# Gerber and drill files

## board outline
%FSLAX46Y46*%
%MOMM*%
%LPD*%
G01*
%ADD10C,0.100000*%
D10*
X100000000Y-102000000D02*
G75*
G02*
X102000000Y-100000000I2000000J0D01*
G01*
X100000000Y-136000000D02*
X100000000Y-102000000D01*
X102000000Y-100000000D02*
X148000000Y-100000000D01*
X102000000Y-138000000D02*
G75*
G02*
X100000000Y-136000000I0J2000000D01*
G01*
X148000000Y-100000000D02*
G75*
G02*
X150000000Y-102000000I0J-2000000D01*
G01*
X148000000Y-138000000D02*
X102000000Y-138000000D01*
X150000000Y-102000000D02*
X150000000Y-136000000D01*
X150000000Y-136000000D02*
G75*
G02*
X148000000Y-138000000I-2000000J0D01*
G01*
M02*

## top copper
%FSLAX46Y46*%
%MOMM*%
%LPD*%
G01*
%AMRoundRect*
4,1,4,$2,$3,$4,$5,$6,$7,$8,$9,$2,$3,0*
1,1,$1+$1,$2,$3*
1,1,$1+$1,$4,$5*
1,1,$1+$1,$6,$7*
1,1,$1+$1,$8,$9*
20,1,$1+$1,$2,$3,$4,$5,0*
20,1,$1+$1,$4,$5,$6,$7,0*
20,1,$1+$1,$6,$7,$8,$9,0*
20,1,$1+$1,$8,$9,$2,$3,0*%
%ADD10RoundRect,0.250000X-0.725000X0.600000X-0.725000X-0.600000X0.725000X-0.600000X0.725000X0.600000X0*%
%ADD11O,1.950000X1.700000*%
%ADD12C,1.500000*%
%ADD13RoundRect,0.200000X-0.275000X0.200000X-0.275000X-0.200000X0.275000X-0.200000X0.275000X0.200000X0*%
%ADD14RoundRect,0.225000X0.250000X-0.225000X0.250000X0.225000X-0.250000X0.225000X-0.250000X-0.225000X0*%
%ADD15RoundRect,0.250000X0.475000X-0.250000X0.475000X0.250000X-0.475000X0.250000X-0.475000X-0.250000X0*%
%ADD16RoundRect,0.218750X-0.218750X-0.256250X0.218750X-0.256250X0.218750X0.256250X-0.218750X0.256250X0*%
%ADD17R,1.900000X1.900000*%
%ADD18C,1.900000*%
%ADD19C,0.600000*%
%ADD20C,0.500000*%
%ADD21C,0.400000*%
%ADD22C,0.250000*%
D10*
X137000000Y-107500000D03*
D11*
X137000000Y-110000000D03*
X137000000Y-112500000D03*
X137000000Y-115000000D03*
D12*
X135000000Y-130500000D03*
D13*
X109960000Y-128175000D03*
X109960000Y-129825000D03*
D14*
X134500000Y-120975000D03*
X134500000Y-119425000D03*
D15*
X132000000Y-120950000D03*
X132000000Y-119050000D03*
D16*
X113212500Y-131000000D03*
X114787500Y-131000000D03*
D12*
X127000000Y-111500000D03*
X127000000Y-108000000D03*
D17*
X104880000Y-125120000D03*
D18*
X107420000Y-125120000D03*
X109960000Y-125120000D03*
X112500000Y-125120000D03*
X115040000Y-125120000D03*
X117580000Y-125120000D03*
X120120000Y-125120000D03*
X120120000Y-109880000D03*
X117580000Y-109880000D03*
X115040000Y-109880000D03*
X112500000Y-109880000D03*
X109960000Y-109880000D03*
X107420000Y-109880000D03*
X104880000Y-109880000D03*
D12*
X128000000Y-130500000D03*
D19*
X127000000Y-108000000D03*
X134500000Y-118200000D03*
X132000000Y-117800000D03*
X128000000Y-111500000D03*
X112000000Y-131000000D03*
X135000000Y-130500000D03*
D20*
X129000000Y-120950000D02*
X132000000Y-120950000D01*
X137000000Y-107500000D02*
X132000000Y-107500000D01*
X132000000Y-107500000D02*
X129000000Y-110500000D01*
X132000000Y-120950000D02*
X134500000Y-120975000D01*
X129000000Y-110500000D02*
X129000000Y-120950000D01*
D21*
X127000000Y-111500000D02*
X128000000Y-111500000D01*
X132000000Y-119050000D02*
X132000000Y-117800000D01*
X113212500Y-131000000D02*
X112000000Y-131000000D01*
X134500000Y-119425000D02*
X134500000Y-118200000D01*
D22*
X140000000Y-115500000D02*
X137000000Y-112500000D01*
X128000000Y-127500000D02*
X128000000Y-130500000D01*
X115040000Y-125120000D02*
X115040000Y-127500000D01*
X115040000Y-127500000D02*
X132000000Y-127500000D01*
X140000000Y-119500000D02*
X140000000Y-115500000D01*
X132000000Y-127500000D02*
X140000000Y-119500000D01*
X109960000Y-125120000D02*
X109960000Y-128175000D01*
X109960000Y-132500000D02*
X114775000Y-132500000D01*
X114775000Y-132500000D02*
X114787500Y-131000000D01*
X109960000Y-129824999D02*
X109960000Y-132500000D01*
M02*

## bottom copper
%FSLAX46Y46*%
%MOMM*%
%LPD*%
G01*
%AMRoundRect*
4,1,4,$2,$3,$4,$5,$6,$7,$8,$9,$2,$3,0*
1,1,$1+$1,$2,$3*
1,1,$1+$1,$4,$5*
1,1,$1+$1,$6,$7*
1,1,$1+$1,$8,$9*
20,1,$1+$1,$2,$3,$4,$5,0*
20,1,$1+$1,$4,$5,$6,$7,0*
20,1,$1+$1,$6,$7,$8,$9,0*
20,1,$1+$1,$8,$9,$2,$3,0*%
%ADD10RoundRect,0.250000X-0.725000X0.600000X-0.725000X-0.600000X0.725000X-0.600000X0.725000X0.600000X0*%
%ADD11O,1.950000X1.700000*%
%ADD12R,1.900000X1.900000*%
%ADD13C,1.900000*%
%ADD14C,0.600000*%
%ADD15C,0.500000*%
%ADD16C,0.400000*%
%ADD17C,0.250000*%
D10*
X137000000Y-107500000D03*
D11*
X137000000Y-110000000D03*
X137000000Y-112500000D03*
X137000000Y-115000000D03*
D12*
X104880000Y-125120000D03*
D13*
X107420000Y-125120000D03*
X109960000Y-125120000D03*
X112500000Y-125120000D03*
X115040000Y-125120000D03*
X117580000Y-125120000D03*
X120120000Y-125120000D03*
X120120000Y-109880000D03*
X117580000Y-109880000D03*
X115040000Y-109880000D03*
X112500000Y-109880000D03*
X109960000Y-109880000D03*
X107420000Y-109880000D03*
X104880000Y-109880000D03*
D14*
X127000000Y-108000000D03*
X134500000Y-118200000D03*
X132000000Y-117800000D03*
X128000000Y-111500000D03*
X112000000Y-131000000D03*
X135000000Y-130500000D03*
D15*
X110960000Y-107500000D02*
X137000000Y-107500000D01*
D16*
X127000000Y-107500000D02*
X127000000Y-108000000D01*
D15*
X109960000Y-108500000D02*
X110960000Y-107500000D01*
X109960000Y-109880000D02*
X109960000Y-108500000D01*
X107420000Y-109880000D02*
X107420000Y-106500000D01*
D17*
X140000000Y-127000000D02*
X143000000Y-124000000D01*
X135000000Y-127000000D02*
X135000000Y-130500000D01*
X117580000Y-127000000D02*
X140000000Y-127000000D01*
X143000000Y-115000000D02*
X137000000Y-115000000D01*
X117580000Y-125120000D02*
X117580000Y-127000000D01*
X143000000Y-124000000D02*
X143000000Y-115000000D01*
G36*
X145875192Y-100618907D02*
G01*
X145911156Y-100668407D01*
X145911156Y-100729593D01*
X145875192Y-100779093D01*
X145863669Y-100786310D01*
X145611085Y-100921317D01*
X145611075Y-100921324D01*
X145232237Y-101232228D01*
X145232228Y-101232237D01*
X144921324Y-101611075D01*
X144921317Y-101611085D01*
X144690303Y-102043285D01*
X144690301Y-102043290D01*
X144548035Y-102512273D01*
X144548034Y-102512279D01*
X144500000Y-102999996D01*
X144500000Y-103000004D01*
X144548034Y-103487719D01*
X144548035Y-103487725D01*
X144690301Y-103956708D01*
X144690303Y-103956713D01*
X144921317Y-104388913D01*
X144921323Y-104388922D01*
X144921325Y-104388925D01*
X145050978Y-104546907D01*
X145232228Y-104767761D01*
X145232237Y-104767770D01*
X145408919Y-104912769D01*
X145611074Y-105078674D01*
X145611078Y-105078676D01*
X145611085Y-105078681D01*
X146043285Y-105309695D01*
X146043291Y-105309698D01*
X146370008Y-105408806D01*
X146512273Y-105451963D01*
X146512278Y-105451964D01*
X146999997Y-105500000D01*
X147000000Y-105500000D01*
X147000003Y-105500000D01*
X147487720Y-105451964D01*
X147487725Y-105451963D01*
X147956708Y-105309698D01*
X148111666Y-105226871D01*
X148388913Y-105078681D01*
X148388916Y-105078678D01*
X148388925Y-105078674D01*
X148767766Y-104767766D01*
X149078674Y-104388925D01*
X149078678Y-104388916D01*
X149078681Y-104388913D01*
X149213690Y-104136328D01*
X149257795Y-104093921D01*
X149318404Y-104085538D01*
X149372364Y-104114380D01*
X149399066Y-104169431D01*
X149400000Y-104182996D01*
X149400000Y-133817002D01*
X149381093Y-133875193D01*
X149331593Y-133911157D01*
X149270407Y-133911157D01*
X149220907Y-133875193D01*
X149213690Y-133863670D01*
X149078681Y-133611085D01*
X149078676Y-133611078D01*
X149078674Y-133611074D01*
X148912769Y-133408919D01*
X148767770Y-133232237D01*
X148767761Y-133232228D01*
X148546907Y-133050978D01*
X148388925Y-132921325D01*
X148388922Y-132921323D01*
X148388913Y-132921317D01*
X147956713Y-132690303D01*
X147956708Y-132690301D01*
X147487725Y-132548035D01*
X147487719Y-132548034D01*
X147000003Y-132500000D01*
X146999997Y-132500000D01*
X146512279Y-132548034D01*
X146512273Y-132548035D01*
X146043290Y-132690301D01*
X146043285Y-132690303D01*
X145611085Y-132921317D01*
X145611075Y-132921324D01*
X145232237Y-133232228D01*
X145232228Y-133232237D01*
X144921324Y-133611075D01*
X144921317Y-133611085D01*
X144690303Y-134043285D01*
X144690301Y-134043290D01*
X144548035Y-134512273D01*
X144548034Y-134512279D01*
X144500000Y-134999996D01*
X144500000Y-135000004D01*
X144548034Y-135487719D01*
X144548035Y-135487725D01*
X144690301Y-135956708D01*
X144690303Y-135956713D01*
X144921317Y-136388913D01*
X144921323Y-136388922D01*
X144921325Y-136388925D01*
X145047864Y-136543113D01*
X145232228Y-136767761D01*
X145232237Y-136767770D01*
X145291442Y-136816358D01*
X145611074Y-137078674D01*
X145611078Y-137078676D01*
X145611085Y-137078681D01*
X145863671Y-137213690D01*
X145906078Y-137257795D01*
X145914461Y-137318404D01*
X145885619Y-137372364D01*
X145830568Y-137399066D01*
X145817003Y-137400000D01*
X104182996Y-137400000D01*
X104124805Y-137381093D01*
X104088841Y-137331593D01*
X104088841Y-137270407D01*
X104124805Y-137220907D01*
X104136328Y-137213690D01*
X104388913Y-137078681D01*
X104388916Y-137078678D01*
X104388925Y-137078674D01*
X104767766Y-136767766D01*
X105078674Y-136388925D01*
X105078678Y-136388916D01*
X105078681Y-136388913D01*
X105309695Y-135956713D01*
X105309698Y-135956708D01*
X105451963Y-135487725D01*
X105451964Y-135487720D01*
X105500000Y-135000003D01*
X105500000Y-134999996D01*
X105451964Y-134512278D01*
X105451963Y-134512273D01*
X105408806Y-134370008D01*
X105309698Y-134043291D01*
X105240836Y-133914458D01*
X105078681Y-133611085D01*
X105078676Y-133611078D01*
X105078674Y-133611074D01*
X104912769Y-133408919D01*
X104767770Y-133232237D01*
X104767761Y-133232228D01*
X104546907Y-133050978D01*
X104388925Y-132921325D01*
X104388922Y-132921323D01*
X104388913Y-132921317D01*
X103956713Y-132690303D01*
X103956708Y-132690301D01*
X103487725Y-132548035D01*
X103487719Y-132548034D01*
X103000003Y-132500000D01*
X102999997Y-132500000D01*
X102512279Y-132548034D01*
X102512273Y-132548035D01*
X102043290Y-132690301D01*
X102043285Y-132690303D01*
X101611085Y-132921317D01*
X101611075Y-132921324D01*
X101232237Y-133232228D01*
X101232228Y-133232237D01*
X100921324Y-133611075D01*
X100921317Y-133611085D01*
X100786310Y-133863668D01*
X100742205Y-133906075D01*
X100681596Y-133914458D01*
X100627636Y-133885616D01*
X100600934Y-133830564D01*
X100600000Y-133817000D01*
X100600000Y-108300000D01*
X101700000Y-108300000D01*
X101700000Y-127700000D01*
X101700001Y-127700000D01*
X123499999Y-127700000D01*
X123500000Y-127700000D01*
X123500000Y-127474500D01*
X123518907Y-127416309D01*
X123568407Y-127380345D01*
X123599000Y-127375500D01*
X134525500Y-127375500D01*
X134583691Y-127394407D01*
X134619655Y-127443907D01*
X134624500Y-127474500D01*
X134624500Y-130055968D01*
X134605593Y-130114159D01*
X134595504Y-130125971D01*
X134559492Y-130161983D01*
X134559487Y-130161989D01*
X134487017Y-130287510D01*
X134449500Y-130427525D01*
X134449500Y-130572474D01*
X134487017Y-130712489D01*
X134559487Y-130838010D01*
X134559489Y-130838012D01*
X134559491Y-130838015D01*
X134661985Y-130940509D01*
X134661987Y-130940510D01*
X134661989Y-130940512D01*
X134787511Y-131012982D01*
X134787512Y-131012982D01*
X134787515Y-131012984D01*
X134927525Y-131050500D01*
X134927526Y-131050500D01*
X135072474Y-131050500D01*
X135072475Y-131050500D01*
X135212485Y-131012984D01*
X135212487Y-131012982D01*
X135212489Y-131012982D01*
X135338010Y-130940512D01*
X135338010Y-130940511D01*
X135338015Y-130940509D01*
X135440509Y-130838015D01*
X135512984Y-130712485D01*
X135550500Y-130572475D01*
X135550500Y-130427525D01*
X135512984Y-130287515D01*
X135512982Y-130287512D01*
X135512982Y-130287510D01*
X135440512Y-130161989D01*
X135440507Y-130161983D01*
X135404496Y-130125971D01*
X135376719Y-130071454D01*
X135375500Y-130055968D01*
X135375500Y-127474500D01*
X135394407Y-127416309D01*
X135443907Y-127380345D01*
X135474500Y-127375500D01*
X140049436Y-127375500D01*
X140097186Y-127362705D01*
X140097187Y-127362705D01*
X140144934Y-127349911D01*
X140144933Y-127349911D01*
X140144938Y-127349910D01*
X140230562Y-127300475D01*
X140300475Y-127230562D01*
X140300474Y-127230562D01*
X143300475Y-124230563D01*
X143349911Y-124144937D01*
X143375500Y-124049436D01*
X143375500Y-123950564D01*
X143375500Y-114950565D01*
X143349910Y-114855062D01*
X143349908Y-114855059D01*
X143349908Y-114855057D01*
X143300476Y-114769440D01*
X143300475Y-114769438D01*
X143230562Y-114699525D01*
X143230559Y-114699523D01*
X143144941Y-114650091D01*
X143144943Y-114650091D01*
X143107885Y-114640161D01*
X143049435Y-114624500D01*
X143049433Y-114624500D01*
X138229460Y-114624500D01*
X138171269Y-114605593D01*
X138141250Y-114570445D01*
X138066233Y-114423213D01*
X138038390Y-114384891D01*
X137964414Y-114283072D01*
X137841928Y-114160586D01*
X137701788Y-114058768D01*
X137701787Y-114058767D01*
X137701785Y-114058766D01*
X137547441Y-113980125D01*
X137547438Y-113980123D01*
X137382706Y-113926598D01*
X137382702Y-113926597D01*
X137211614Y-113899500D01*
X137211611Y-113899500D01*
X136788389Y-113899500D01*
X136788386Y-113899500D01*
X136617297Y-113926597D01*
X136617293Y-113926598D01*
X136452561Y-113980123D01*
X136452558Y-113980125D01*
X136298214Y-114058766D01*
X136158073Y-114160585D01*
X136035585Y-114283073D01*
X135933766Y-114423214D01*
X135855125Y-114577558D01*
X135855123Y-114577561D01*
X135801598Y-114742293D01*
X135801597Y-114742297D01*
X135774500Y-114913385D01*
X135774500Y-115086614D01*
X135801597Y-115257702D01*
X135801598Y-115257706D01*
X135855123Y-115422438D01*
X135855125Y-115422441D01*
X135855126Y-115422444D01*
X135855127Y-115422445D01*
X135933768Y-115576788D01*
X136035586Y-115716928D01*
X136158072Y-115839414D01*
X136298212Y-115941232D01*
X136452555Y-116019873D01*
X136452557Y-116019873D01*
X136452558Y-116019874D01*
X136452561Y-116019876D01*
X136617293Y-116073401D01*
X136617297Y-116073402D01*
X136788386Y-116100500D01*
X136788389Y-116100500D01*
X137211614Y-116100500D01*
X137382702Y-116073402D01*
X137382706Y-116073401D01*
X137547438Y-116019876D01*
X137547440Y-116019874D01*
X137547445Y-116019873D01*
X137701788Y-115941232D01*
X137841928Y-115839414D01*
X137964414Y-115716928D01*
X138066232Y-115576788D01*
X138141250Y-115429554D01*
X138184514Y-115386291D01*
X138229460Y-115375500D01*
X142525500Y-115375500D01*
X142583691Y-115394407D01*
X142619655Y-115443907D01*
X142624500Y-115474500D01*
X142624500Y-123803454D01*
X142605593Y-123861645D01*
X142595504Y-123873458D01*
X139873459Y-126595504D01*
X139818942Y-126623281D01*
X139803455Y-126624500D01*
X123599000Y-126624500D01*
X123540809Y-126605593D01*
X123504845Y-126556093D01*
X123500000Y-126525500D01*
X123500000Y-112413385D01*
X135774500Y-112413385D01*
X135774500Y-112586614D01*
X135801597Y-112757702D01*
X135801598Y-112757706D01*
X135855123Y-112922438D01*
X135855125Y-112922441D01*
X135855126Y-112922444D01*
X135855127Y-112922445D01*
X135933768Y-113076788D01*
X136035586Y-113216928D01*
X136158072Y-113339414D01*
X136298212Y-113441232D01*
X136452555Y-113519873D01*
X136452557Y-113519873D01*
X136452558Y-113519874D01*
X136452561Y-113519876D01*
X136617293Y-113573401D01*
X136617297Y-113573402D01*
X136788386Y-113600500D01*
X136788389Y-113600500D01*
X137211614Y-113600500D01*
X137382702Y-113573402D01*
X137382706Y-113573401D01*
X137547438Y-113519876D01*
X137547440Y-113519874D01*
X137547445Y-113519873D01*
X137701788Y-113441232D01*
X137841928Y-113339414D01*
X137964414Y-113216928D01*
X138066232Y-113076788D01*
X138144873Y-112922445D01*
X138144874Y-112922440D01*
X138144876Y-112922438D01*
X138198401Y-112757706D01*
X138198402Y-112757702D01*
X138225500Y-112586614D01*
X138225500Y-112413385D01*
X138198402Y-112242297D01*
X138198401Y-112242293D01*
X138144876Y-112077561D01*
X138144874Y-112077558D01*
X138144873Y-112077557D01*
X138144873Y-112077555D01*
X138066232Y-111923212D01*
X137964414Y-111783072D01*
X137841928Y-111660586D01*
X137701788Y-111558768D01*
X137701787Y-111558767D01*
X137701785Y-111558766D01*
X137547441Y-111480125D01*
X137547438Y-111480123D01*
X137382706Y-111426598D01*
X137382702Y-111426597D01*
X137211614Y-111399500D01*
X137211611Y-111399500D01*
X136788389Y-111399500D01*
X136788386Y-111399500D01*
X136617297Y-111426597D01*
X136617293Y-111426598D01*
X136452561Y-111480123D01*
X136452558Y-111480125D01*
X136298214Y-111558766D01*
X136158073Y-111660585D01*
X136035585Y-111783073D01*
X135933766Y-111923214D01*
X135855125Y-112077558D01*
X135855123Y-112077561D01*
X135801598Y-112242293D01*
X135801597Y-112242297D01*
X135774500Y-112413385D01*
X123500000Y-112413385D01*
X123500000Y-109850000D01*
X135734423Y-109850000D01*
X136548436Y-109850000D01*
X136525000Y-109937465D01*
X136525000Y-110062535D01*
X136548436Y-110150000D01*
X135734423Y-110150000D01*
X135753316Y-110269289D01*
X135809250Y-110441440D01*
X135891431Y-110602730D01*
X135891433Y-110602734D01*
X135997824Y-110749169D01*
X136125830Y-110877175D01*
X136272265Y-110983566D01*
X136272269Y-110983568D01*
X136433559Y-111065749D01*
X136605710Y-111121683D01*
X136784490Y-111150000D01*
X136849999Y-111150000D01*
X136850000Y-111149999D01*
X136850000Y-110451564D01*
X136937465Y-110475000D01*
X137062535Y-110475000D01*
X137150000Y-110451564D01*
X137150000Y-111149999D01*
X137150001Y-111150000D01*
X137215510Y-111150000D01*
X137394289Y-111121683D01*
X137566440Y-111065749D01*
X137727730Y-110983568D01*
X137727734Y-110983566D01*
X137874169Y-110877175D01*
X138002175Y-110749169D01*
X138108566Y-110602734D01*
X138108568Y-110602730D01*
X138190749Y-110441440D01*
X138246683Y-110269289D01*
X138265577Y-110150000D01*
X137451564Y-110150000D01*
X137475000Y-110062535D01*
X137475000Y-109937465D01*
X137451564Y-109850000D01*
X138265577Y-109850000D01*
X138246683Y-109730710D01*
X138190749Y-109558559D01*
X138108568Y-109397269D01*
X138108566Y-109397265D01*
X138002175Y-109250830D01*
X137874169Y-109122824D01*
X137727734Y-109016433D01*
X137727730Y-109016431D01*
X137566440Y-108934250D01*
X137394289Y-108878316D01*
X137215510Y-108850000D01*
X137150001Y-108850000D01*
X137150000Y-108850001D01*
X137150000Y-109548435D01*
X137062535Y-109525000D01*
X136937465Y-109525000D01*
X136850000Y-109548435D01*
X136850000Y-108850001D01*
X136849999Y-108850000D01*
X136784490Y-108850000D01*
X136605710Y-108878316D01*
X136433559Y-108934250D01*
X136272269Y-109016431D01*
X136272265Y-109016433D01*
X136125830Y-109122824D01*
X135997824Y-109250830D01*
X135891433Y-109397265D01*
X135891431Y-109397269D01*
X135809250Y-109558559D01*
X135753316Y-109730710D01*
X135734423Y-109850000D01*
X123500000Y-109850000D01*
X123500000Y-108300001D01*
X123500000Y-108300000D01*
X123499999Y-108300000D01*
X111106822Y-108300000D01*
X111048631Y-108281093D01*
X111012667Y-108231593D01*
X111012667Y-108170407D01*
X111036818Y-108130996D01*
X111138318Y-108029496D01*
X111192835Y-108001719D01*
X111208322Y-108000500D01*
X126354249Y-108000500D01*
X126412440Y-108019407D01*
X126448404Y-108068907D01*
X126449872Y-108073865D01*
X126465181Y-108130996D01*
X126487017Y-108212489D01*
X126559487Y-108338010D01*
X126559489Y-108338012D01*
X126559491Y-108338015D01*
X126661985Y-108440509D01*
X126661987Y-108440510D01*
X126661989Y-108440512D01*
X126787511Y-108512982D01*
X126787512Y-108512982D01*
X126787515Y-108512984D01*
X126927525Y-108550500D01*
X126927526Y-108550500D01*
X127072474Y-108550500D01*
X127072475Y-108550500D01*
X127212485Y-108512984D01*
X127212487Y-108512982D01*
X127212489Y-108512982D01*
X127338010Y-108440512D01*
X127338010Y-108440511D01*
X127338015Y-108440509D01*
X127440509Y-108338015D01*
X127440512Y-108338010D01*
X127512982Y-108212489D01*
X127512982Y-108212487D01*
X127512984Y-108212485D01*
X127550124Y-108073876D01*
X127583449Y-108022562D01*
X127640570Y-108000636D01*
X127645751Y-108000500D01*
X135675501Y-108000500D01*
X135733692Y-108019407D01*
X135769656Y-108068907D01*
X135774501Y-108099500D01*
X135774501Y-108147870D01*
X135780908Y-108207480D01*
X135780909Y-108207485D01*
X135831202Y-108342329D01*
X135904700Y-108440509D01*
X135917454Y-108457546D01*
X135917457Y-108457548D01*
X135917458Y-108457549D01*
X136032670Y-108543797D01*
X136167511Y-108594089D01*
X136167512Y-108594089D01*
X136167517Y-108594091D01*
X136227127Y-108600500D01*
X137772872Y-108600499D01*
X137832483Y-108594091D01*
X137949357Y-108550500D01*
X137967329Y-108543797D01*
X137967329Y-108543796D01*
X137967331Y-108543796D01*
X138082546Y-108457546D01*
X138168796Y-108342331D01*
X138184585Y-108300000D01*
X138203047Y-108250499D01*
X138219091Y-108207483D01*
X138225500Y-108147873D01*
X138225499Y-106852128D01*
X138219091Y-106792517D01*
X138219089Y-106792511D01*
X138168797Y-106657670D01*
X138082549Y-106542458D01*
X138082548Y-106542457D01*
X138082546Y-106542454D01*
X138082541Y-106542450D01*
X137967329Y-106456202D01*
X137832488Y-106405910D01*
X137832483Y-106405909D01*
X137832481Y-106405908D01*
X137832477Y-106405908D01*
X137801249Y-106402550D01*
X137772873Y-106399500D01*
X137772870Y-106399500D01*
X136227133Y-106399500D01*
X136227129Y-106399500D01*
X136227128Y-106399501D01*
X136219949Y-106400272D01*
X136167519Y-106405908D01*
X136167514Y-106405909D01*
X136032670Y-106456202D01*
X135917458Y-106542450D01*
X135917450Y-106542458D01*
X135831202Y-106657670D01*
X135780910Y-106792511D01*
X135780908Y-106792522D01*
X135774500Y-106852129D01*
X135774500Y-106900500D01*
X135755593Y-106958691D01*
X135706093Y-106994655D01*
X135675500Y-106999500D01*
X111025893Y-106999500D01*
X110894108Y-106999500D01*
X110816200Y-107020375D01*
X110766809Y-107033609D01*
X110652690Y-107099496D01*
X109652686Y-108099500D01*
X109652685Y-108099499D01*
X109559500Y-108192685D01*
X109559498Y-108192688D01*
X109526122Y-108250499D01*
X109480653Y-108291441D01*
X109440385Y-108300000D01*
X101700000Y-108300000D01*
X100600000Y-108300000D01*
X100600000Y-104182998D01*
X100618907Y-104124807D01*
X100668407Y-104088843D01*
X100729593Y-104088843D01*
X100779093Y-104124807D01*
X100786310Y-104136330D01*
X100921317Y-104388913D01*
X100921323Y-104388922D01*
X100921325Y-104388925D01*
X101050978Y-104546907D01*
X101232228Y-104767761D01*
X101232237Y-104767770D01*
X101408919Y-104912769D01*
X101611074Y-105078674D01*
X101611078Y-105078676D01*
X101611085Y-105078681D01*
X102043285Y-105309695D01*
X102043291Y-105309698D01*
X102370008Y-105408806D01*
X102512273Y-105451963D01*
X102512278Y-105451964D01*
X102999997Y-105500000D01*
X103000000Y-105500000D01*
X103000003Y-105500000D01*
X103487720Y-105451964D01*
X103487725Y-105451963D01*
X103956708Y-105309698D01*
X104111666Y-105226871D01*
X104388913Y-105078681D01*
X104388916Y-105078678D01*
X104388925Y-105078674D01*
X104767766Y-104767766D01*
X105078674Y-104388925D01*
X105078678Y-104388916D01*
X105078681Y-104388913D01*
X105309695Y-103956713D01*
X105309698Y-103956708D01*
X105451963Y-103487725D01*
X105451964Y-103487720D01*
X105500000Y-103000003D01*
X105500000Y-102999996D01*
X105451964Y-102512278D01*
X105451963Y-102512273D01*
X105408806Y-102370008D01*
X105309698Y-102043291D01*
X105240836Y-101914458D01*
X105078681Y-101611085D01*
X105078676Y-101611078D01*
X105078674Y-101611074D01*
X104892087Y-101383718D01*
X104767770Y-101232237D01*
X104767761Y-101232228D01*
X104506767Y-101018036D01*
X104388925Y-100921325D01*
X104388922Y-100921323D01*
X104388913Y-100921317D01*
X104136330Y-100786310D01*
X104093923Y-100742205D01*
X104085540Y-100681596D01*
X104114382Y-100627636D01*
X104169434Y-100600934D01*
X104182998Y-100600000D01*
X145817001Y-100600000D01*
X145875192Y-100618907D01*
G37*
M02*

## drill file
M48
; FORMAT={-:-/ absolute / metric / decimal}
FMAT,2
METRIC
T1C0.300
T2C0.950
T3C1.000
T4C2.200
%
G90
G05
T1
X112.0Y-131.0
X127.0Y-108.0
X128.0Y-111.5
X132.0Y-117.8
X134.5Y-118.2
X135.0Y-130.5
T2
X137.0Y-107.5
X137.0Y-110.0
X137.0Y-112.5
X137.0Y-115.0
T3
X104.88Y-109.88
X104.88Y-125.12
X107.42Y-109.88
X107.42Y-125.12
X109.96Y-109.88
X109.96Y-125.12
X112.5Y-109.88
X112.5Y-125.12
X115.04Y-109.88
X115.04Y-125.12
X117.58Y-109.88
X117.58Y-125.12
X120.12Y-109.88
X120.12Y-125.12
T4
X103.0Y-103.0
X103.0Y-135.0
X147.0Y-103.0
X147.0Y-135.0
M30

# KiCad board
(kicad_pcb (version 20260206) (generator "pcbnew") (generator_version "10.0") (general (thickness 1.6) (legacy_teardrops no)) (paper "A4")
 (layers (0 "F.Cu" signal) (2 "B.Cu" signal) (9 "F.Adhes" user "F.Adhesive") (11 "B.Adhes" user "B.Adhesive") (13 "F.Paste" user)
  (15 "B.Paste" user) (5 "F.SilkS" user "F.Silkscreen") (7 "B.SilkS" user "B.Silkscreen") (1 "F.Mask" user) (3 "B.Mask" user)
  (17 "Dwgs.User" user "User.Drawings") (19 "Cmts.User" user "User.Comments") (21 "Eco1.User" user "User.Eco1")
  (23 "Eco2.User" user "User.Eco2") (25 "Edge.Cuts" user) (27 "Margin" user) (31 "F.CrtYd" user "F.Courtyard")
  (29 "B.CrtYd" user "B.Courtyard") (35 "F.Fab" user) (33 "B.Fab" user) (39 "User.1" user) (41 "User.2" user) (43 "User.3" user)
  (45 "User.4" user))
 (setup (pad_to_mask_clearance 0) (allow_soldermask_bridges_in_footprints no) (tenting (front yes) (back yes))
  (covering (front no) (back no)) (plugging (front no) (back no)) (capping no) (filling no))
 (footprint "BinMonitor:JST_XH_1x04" (layer "F.Cu") (at 137 107.5 -90)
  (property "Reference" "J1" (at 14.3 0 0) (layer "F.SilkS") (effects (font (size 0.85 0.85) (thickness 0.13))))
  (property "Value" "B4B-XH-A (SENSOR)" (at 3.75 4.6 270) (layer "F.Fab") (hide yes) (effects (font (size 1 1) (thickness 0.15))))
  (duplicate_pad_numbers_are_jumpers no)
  (pad "1" thru_hole roundrect (at 0 0 270) (size 1.7 1.95) (drill 0.95) (layers "*.Cu" "*.Mask") (remove_unused_layers no)
   (roundrect_rratio 0.147059) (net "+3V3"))
  (pad "2" thru_hole oval (at 2.5 0 270) (size 1.7 1.95) (drill 0.95) (layers "*.Cu" "*.Mask") (remove_unused_layers no) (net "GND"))
  (pad "3" thru_hole oval (at 5 0 270) (size 1.7 1.95) (drill 0.95) (layers "*.Cu" "*.Mask") (remove_unused_layers no) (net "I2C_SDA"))
  (pad "4" thru_hole oval (at 7.5 0 270) (size 1.7 1.95) (drill 0.95) (layers "*.Cu" "*.Mask") (remove_unused_layers no) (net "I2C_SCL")))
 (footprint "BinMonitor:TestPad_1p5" (layer "F.Cu") (at 135 130.5)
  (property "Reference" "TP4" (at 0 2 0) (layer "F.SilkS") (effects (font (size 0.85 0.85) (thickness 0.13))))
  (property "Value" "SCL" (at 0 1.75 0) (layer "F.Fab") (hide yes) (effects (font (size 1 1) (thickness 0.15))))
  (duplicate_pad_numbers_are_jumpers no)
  (pad "1" smd circle (at 0 0) (size 1.5 1.5) (layers "F.Cu" "F.Mask") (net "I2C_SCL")))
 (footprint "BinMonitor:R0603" (layer "F.Cu") (at 109.96 129 -90)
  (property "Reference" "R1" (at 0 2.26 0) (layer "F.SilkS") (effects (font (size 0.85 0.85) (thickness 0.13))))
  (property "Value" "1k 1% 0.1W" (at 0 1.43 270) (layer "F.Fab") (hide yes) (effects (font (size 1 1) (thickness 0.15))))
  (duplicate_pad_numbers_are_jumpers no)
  (pad "1" smd roundrect (at -0.825 0 270) (size 0.8 0.95) (layers "F.Cu" "F.Mask" "F.Paste") (roundrect_rratio 0.25) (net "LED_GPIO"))
  (pad "2" smd roundrect (at 0.825 0 270) (size 0.8 0.95) (layers "F.Cu" "F.Mask" "F.Paste") (roundrect_rratio 0.25) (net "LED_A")))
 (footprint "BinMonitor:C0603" (layer "F.Cu") (at 134.5 120.2 90)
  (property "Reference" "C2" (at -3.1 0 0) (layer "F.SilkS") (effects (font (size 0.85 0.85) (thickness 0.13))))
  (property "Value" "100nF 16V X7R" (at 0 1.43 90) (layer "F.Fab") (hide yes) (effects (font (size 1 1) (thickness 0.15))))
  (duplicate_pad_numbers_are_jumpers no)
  (pad "1" smd roundrect (at -0.775 0 90) (size 0.9 0.95) (layers "F.Cu" "F.Mask" "F.Paste") (roundrect_rratio 0.25) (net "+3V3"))
  (pad "2" smd roundrect (at 0.775 0 90) (size 0.9 0.95) (layers "F.Cu" "F.Mask" "F.Paste") (roundrect_rratio 0.25) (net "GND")))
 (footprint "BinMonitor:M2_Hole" (layer "F.Cu") (at 103 135)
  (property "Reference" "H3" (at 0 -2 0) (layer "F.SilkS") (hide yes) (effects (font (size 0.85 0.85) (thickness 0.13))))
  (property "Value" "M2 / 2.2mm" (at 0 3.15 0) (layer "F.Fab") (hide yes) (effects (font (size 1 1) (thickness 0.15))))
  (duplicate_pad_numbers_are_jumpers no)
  (pad "" np_thru_hole circle (at 0 0) (size 2.2 2.2) (drill 2.2) (layers "*.Cu" "*.Mask")))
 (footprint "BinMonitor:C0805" (layer "F.Cu") (at 132 120 90)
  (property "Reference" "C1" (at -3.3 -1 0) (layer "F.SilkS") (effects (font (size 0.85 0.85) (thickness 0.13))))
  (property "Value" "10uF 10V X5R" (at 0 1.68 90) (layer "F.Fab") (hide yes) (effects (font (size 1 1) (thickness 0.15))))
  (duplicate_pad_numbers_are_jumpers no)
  (pad "1" smd roundrect (at -0.95 0 90) (size 1 1.45) (layers "F.Cu" "F.Mask" "F.Paste") (roundrect_rratio 0.25) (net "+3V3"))
  (pad "2" smd roundrect (at 0.95 0 90) (size 1 1.45) (layers "F.Cu" "F.Mask" "F.Paste") (roundrect_rratio 0.25) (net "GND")))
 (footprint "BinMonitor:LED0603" (layer "F.Cu") (at 114 131)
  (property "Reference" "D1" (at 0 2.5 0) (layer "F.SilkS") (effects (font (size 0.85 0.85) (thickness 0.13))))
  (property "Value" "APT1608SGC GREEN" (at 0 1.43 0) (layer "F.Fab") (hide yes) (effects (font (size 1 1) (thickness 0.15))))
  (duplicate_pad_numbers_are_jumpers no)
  (pad "1" smd roundrect (at -0.7875 0) (size 0.875 0.95) (layers "F.Cu" "F.Mask" "F.Paste") (roundrect_rratio 0.25) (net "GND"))
  (pad "2" smd roundrect (at 0.7875 0) (size 0.875 0.95) (layers "F.Cu" "F.Mask" "F.Paste") (roundrect_rratio 0.25) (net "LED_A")))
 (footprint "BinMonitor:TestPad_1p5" (layer "F.Cu") (at 127 111.5)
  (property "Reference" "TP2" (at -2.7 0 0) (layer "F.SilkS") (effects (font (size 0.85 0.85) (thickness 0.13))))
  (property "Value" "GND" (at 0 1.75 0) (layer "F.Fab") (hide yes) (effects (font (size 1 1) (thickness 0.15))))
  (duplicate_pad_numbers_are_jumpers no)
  (pad "1" smd circle (at 0 0) (size 1.5 1.5) (layers "F.Cu" "F.Mask") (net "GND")))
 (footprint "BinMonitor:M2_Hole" (layer "F.Cu") (at 147 103)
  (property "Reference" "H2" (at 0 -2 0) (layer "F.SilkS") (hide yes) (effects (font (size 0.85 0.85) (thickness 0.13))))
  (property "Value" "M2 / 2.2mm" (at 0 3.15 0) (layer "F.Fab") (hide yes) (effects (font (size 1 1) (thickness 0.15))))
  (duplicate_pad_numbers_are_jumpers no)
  (pad "" np_thru_hole circle (at 0 0) (size 2.2 2.2) (drill 2.2) (layers "*.Cu" "*.Mask")))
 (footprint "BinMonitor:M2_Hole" (layer "F.Cu") (at 147 135)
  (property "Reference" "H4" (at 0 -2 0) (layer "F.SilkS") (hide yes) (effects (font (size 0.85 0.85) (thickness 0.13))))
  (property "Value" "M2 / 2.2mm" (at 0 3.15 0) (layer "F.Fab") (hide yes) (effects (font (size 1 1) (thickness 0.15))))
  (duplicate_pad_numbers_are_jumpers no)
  (pad "" np_thru_hole circle (at 0 0) (size 2.2 2.2) (drill 2.2) (layers "*.Cu" "*.Mask")))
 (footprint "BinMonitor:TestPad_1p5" (layer "F.Cu") (at 127 108)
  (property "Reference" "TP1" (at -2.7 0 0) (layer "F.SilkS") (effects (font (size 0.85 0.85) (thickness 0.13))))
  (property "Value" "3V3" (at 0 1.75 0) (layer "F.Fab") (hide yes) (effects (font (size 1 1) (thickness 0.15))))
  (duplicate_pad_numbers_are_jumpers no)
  (pad "1" smd circle (at 0 0) (size 1.5 1.5) (layers "F.Cu" "F.Mask") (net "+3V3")))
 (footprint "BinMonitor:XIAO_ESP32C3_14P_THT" (layer "F.Cu") (at 112.5 117.5 180)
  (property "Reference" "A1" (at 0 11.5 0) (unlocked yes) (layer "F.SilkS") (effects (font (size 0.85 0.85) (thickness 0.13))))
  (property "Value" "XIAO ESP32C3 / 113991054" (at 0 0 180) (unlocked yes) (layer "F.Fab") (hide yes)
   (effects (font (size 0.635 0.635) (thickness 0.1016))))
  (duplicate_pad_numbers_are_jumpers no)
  (pad "1" thru_hole rect (at 7.62 -7.62 270) (size 1.9 1.9) (drill 1) (layers "*.Cu" "*.Mask") (remove_unused_layers no)
   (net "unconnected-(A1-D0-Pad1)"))
  (pad "2" thru_hole circle (at 5.08 -7.62 270) (size 1.9 1.9) (drill 1) (layers "*.Cu" "*.Mask") (remove_unused_layers no)
   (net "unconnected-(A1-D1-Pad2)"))
  (pad "3" thru_hole circle (at 2.54 -7.62 270) (size 1.9 1.9) (drill 1) (layers "*.Cu" "*.Mask") (remove_unused_layers no) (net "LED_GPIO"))
  (pad "4" thru_hole circle (at 0 -7.62 270) (size 1.9 1.9) (drill 1) (layers "*.Cu" "*.Mask") (remove_unused_layers no)
   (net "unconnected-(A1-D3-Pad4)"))
  (pad "5" thru_hole circle (at -2.54 -7.62 270) (size 1.9 1.9) (drill 1) (layers "*.Cu" "*.Mask") (remove_unused_layers no) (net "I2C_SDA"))
  (pad "6" thru_hole circle (at -5.08 -7.62 270) (size 1.9 1.9) (drill 1) (layers "*.Cu" "*.Mask") (remove_unused_layers no) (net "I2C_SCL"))
  (pad "7" thru_hole circle (at -7.62 -7.62 270) (size 1.9 1.9) (drill 1) (layers "*.Cu" "*.Mask") (remove_unused_layers no)
   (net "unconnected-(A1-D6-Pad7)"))
  (pad "8" thru_hole circle (at -7.62 7.62 90) (size 1.9 1.9) (drill 1) (layers "*.Cu" "*.Mask") (remove_unused_layers no)
   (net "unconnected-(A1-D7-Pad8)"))
  (pad "9" thru_hole circle (at -5.08 7.62 90) (size 1.9 1.9) (drill 1) (layers "*.Cu" "*.Mask") (remove_unused_layers no)
   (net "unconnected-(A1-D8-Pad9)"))
  (pad "10" thru_hole circle (at -2.54 7.62 90) (size 1.9 1.9) (drill 1) (layers "*.Cu" "*.Mask") (remove_unused_layers no)
   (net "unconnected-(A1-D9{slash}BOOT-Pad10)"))
  (pad "11" thru_hole circle (at 0 7.62 90) (size 1.9 1.9) (drill 1) (layers "*.Cu" "*.Mask") (remove_unused_layers no)
   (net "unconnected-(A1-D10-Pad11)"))
  (pad "12" thru_hole circle (at 2.54 7.62 90) (size 1.9 1.9) (drill 1) (layers "*.Cu" "*.Mask") (remove_unused_layers no) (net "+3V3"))
  (pad "13" thru_hole circle (at 5.08 7.62 90) (size 1.9 1.9) (drill 1) (layers "*.Cu" "*.Mask") (remove_unused_layers no) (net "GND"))
  (pad "14" thru_hole circle (at 7.62 7.62 90) (size 1.9 1.9) (drill 1) (layers "*.Cu" "*.Mask") (remove_unused_layers no)
   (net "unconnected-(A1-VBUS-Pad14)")))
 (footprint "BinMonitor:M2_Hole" (layer "F.Cu") (at 103 103)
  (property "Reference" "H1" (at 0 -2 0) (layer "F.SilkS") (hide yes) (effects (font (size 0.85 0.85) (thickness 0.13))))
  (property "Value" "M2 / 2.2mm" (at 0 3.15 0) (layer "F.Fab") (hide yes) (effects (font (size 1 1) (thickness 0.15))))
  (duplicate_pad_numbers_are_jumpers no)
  (pad "" np_thru_hole circle (at 0 0) (size 2.2 2.2) (drill 2.2) (layers "*.Cu" "*.Mask")))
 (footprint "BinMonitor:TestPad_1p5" (layer "F.Cu") (at 128 130.5)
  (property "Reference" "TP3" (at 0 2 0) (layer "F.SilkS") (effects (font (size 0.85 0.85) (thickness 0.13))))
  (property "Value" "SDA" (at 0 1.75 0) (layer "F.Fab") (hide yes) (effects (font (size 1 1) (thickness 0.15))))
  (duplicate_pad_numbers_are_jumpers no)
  (pad "1" smd circle (at 0 0) (size 1.5 1.5) (layers "F.Cu" "F.Mask") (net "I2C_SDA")))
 (gr_arc (start 100 102) (mid 100.585786 100.585786) (end 102 100) (stroke (width 0.1) (type default)) (layer "Edge.Cuts"))
 (gr_line (start 100 136) (end 100 102) (stroke (width 0.1) (type default)) (layer "Edge.Cuts"))
 (gr_line (start 102 100) (end 148 100) (stroke (width 0.1) (type default)) (layer "Edge.Cuts"))
 (gr_arc (start 102 138) (mid 100.585786 137.414214) (end 100 136) (stroke (width 0.1) (type default)) (layer "Edge.Cuts"))
 (gr_arc (start 148 100) (mid 149.414214 100.585786) (end 150 102) (stroke (width 0.1) (type default)) (layer "Edge.Cuts"))
 (gr_line (start 148 138) (end 102 138) (stroke (width 0.1) (type default)) (layer "Edge.Cuts"))
 (gr_line (start 150 102) (end 150 136) (stroke (width 0.1) (type default)) (layer "Edge.Cuts"))
 (gr_arc (start 150 136) (mid 149.414214 137.414214) (end 148 138) (stroke (width 0.1) (type default)) (layer "Edge.Cuts"))
 (segment (start 129 120.95) (end 132 120.95) (width 0.5) (layer "F.Cu") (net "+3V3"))
 (segment (start 137 107.5) (end 132 107.5) (width 0.5) (layer "F.Cu") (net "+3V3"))
 (segment (start 132 107.5) (end 129 110.5) (width 0.5) (layer "F.Cu") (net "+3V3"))
 (segment (start 132 120.95) (end 134.5 120.975) (width 0.5) (layer "F.Cu") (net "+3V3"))
 (segment (start 129 110.5) (end 129 120.95) (width 0.5) (layer "F.Cu") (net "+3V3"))
 (via (at 127 108) (size 0.6) (drill 0.3) (layers "F.Cu" "B.Cu") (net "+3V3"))
 (segment (start 110.96 107.5) (end 137 107.5) (width 0.5) (layer "B.Cu") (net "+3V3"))
 (segment (start 127 107.5) (end 127 108) (width 0.4) (layer "B.Cu") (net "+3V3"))
 (segment (start 109.96 108.5) (end 110.96 107.5) (width 0.5) (layer "B.Cu") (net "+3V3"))
 (segment (start 109.96 109.88) (end 109.96 108.5) (width 0.5) (layer "B.Cu") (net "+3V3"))
 (segment (start 127 111.5) (end 128 111.5) (width 0.4) (layer "F.Cu") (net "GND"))
 (segment (start 132 119.05) (end 132 117.8) (width 0.4) (layer "F.Cu") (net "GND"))
 (segment (start 113.2125 131) (end 112 131) (width 0.4) (layer "F.Cu") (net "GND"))
 (segment (start 134.5 119.425) (end 134.5 118.2) (width 0.4) (layer "F.Cu") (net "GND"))
 (via (at 134.5 118.2) (size 0.6) (drill 0.3) (layers "F.Cu" "B.Cu") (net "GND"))
 (via (at 132 117.8) (size 0.6) (drill 0.3) (layers "F.Cu" "B.Cu") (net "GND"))
 (via (at 128 111.5) (size 0.6) (drill 0.3) (layers "F.Cu" "B.Cu") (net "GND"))
 (via (at 112 131) (size 0.6) (drill 0.3) (layers "F.Cu" "B.Cu") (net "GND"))
 (segment (start 107.42 109.88) (end 107.42 106.5) (width 0.5) (layer "B.Cu") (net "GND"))
 (segment (start 140 115.5) (end 137 112.5) (width 0.25) (layer "F.Cu") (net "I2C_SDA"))
 (segment (start 128 127.5) (end 128 130.5) (width 0.25) (layer "F.Cu") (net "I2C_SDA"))
 (segment (start 115.04 125.12) (end 115.04 127.5) (width 0.25) (layer "F.Cu") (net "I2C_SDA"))
 (segment (start 115.04 127.5) (end 132 127.5) (width 0.25) (layer "F.Cu") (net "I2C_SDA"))
 (segment (start 140 119.5) (end 140 115.5) (width 0.25) (layer "F.Cu") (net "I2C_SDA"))
 (segment (start 132 127.5) (end 140 119.5) (width 0.25) (layer "F.Cu") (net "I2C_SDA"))
 (via (at 135 130.5) (size 0.6) (drill 0.3) (layers "F.Cu" "B.Cu") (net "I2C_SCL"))
 (segment (start 140 127) (end 143 124) (width 0.25) (layer "B.Cu") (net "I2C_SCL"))
 (segment (start 135 127) (end 135 130.5) (width 0.25) (layer "B.Cu") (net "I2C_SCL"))
 (segment (start 117.58 127) (end 140 127) (width 0.25) (layer "B.Cu") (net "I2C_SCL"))
 (segment (start 143 115) (end 137 115) (width 0.25) (layer "B.Cu") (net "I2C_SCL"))
 (segment (start 117.58 125.12) (end 117.58 127) (width 0.25) (layer "B.Cu") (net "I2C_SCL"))
 (segment (start 143 124) (end 143 115) (width 0.25) (layer "B.Cu") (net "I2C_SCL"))
 (segment (start 109.96 125.12) (end 109.96 128.175) (width 0.25) (layer "F.Cu") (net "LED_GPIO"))
 (segment (start 109.96 132.5) (end 114.775 132.5) (width 0.25) (layer "F.Cu") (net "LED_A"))
 (segment (start 114.775 132.5) (end 114.7875 131) (width 0.25) (layer "F.Cu") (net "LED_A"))
 (segment (start 109.96 129.824999) (end 109.96 132.5) (width 0.25) (layer "F.Cu") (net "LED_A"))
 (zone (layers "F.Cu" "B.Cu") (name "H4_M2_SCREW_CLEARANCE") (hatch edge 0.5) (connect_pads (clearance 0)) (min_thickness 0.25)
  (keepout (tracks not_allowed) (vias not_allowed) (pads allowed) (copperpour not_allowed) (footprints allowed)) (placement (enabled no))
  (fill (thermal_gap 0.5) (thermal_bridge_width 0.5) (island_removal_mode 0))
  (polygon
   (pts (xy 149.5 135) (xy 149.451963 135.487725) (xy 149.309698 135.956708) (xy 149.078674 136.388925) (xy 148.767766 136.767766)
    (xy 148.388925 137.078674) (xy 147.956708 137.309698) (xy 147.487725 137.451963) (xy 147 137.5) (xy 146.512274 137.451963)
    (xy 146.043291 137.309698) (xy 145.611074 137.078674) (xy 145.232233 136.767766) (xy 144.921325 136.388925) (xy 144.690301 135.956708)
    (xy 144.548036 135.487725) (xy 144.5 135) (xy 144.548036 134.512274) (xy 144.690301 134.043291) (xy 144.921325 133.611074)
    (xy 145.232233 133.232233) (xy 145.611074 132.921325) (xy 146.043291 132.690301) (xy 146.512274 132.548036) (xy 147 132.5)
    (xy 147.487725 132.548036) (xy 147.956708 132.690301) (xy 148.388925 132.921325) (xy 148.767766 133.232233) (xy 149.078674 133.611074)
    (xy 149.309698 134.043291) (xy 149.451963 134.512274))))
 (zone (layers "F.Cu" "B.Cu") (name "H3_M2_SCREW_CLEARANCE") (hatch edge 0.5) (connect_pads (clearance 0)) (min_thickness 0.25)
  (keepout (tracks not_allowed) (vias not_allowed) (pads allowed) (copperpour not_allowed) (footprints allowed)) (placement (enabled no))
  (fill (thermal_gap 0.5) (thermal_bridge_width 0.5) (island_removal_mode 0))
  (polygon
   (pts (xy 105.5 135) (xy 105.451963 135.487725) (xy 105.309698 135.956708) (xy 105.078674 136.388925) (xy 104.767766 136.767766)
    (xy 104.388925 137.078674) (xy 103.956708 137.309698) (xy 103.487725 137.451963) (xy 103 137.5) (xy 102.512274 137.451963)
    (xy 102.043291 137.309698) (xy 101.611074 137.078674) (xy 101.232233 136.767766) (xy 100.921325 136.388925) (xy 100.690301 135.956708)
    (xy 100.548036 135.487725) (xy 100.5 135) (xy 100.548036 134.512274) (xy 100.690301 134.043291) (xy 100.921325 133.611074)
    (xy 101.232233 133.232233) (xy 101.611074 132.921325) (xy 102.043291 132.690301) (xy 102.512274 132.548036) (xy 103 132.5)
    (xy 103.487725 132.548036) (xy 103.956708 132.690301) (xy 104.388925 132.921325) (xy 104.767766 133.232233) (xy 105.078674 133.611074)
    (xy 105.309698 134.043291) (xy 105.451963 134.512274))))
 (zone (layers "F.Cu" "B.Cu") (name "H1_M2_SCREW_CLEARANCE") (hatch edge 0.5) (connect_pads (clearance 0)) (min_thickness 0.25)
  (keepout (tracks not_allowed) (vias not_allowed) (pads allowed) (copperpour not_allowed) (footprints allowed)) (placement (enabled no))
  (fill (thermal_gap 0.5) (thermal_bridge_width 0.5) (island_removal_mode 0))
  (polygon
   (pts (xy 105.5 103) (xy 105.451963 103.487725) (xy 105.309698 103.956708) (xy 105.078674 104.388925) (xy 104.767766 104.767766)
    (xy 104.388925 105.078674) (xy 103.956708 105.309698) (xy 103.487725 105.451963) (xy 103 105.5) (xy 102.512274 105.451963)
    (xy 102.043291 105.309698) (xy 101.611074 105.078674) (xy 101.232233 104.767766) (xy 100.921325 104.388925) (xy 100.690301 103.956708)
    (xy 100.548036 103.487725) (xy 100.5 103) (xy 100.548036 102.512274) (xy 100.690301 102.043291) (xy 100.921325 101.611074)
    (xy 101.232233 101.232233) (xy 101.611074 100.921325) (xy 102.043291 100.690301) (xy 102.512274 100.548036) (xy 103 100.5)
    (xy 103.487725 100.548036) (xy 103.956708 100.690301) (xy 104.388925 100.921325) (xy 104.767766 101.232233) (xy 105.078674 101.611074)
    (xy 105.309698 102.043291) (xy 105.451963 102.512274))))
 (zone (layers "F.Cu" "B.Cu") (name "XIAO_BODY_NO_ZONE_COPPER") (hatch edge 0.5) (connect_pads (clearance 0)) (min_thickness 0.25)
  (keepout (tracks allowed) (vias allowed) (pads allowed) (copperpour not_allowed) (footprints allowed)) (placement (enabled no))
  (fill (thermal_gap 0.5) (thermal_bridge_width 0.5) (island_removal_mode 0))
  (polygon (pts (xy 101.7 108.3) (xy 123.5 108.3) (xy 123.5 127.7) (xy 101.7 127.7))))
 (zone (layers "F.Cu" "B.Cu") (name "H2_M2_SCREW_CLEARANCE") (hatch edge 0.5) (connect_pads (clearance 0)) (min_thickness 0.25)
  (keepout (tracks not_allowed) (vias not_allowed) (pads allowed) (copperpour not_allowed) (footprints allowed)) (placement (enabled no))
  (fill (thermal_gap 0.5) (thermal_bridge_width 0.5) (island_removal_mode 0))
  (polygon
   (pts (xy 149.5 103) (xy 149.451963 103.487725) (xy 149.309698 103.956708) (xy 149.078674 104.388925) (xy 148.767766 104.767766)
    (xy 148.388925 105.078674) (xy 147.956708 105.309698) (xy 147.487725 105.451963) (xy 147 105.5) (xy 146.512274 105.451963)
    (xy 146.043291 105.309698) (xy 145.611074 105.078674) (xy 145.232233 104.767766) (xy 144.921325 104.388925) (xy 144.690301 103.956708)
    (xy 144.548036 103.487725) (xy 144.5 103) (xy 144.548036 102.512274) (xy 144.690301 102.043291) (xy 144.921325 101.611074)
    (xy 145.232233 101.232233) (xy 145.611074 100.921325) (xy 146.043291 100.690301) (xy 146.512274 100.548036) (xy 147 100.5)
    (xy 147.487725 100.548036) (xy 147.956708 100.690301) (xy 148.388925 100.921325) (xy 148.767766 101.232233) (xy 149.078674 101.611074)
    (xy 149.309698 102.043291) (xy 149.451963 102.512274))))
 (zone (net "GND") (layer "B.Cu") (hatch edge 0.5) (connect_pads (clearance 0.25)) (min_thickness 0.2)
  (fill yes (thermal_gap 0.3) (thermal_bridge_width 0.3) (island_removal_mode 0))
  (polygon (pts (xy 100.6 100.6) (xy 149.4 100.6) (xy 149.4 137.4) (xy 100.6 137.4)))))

